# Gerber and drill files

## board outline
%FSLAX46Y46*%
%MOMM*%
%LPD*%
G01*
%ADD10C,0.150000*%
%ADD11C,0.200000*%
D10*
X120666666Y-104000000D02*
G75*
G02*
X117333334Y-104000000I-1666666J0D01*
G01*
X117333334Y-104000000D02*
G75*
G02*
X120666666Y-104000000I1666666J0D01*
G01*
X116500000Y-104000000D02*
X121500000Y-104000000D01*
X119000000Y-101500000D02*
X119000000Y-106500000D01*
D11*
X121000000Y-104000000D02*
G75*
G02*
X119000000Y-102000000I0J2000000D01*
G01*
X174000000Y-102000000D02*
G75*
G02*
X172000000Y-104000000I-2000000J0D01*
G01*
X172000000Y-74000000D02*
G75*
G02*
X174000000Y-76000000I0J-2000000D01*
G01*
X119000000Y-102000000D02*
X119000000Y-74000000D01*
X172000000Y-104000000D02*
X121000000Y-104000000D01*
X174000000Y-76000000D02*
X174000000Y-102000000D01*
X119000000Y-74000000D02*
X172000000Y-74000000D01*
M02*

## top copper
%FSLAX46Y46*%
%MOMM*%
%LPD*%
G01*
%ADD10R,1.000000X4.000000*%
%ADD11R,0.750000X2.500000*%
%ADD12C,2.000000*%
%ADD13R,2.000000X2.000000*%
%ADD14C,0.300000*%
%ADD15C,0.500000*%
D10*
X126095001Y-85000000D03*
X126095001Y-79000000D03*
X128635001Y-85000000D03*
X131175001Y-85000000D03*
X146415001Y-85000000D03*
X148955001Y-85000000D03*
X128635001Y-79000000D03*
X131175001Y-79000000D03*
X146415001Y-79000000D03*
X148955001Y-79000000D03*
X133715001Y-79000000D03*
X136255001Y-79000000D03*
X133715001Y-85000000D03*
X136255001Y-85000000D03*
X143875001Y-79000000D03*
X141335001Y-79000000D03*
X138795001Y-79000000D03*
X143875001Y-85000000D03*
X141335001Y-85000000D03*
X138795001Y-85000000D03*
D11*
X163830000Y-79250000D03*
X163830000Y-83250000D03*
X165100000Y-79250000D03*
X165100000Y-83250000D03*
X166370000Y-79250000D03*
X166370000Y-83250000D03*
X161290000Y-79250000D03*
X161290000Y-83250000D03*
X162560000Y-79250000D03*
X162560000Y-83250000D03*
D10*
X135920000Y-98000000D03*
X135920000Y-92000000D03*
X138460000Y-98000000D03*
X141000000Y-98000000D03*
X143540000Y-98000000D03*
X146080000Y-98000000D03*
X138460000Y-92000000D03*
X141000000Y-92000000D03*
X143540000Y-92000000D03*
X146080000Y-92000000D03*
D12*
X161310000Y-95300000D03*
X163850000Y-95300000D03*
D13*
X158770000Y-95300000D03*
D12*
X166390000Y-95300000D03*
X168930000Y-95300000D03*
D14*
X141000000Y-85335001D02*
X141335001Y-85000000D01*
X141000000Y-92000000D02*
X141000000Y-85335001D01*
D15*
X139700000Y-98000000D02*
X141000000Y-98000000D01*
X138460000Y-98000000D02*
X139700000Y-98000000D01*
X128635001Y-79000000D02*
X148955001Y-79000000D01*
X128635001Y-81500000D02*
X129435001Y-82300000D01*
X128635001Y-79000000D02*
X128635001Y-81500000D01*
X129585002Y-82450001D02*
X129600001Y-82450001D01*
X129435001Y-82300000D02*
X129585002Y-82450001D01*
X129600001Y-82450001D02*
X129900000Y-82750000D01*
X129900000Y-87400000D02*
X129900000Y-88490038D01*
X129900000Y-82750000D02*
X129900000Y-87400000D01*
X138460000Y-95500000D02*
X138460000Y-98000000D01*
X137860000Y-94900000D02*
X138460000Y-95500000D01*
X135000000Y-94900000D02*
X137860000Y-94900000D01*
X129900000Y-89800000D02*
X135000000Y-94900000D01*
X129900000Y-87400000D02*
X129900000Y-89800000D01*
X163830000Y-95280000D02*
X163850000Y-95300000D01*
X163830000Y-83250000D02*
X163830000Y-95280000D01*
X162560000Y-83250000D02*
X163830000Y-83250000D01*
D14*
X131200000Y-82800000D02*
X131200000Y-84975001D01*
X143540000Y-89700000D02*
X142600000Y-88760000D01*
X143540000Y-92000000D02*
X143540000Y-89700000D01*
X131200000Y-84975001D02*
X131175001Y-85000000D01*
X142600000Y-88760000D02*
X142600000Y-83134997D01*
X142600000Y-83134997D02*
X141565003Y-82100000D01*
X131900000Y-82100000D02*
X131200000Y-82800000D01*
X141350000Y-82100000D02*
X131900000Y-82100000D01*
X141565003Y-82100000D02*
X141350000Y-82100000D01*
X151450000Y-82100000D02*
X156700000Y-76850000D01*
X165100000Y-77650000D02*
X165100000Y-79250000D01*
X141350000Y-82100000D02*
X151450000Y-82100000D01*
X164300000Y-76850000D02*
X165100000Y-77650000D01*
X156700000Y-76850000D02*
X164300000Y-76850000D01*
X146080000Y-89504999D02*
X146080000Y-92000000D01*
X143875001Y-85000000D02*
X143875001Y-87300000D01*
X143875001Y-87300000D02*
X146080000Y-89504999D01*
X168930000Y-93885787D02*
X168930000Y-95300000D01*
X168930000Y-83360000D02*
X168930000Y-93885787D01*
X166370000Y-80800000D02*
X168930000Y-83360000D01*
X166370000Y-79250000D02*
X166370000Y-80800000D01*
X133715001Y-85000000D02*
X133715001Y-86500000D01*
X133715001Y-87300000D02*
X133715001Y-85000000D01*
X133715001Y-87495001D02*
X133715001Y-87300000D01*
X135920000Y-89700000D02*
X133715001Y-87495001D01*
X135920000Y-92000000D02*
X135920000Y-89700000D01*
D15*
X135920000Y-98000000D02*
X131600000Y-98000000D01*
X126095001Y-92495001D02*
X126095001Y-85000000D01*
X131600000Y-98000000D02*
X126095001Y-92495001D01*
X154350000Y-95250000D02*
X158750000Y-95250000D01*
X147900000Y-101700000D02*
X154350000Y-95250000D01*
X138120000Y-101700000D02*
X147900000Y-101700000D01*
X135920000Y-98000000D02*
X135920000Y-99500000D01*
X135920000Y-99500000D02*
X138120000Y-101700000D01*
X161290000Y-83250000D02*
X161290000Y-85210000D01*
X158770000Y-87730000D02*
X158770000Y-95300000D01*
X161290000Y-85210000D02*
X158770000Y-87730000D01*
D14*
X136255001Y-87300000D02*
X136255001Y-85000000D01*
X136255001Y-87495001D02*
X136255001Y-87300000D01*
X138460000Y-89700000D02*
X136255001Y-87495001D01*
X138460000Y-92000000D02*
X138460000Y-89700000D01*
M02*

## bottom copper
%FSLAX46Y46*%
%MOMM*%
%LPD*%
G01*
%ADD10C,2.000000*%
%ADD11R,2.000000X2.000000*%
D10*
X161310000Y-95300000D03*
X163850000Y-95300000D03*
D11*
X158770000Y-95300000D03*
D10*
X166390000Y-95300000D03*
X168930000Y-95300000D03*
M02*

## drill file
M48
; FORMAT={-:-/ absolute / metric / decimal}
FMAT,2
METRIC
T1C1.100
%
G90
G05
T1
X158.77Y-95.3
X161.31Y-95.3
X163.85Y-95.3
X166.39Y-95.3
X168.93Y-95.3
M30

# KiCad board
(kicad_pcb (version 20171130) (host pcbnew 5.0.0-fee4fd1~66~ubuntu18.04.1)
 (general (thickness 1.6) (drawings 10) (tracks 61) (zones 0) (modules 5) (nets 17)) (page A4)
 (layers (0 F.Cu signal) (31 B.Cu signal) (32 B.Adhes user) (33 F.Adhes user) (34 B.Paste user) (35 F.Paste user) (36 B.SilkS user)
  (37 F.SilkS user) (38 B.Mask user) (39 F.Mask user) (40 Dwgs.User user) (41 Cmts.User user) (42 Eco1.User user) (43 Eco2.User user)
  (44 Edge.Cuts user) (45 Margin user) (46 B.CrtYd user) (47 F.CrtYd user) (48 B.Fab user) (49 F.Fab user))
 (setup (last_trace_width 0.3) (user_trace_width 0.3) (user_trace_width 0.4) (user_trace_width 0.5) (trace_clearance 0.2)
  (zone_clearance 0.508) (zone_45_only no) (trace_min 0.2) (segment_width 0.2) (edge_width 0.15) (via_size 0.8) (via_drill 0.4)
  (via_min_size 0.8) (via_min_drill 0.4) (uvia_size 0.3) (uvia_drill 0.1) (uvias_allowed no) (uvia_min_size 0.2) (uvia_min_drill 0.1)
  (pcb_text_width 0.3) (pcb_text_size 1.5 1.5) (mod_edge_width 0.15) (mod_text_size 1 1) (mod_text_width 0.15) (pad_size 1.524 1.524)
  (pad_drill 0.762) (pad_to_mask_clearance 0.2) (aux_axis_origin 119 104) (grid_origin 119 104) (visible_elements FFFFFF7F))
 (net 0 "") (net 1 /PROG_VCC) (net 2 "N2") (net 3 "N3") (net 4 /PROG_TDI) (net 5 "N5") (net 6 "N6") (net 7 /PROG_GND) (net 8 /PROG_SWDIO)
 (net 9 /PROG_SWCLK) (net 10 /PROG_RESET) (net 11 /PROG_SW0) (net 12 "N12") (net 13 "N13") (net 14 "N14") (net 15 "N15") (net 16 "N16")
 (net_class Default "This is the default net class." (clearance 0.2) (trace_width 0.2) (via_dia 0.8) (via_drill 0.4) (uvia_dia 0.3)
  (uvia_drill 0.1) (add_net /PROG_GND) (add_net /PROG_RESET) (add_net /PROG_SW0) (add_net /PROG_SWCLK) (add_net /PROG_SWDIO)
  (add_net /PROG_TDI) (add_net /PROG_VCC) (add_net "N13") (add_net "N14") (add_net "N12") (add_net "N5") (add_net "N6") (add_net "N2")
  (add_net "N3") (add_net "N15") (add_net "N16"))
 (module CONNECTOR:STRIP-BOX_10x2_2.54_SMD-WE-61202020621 (layer F.Cu) (at 137.525001 82)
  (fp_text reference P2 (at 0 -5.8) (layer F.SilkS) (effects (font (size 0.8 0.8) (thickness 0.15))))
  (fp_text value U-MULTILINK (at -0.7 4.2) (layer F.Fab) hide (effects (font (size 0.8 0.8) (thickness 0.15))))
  (pad 1 smd rect (at -11.43 3) (size 1 4) (layers F.Cu F.Paste F.Mask) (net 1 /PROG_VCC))
  (pad 2 smd rect (at -11.43 -3) (size 1 4) (layers F.Cu F.Paste F.Mask) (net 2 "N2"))
  (pad 3 smd rect (at -8.89 3) (size 1 4) (layers F.Cu F.Paste F.Mask) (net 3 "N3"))
  (pad 5 smd rect (at -6.35 3) (size 1 4) (layers F.Cu F.Paste F.Mask) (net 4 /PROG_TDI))
  (pad 17 smd rect (at 8.89 3) (size 1 4) (layers F.Cu F.Paste F.Mask) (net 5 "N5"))
  (pad 19 smd rect (at 11.43 3) (size 1 4) (layers F.Cu F.Paste F.Mask) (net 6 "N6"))
  (pad 4 smd rect (at -8.89 -3) (size 1 4) (layers F.Cu F.Paste F.Mask) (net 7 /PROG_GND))
  (pad 6 smd rect (at -6.35 -3) (size 1 4) (layers F.Cu F.Paste F.Mask) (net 7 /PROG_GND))
  (pad 18 smd rect (at 8.89 -3) (size 1 4) (layers F.Cu F.Paste F.Mask) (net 7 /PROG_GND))
  (pad 20 smd rect (at 11.43 -3) (size 1 4) (layers F.Cu F.Paste F.Mask) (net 7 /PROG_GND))
  (pad 8 smd rect (at -3.81 -3) (size 1 4) (layers F.Cu F.Paste F.Mask) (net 7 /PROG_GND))
  (pad 10 smd rect (at -1.27 -3) (size 1 4) (layers F.Cu F.Paste F.Mask) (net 7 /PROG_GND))
  (pad 7 smd rect (at -3.81 3) (size 1 4) (layers F.Cu F.Paste F.Mask) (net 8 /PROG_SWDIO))
  (pad 9 smd rect (at -1.27 3) (size 1 4) (layers F.Cu F.Paste F.Mask) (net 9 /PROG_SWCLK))
  (pad 16 smd rect (at 6.35 -3) (size 1 4) (layers F.Cu F.Paste F.Mask) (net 7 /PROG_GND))
  (pad 14 smd rect (at 3.81 -3) (size 1 4) (layers F.Cu F.Paste F.Mask) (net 7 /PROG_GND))
  (pad 12 smd rect (at 1.27 -3) (size 1 4) (layers F.Cu F.Paste F.Mask) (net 7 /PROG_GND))
  (pad 15 smd rect (at 6.35 3) (size 1 4) (layers F.Cu F.Paste F.Mask) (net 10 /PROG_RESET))
  (pad 13 smd rect (at 3.81 3) (size 1 4) (layers F.Cu F.Paste F.Mask) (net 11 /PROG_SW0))
  (pad 11 smd rect (at 1.27 3) (size 1 4) (layers F.Cu F.Paste F.Mask) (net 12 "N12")))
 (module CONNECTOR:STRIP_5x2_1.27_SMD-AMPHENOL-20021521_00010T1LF (layer F.Cu) (at 163.83 81.25)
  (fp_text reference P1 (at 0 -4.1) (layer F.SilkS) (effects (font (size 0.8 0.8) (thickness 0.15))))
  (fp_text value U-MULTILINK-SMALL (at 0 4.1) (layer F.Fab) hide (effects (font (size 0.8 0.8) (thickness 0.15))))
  (pad 6 smd rect (at 0 -2) (size 0.75 2.5) (layers F.Cu F.Paste F.Mask) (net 11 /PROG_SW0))
  (pad 5 smd rect (at 0 2) (size 0.75 2.5) (layers F.Cu F.Paste F.Mask) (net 7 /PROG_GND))
  (pad 8 smd rect (at 1.27 -2) (size 0.75 2.5) (layers F.Cu F.Paste F.Mask) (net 4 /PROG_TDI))
  (pad 7 smd rect (at 1.27 2) (size 0.75 2.5) (layers F.Cu F.Paste F.Mask) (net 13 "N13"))
  (pad 10 smd rect (at 2.54 -2) (size 0.75 2.5) (layers F.Cu F.Paste F.Mask) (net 10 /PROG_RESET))
  (pad 9 smd rect (at 2.54 2) (size 0.75 2.5) (layers F.Cu F.Paste F.Mask) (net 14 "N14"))
  (pad 2 smd rect (at -2.54 -2) (size 0.75 2.5) (layers F.Cu F.Paste F.Mask) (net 8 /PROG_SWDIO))
  (pad 1 smd rect (at -2.54 2) (size 0.75 2.5) (layers F.Cu F.Paste F.Mask) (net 1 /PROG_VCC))
  (pad 4 smd rect (at -1.27 -2) (size 0.75 2.5) (layers F.Cu F.Paste F.Mask) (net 9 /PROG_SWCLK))
  (pad 3 smd rect (at -1.27 2) (size 0.75 2.5) (layers F.Cu F.Paste F.Mask) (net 7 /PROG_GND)))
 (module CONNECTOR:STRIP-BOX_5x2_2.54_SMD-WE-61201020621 (layer F.Cu) (at 141 95)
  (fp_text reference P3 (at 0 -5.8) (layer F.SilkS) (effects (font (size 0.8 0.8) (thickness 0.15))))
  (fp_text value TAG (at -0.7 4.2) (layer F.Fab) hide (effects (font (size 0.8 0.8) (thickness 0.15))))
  (pad 1 smd rect (at -5.08 3) (size 1 4) (layers F.Cu F.Paste F.Mask) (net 1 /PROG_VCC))
  (pad 2 smd rect (at -5.08 -3) (size 1 4) (layers F.Cu F.Paste F.Mask) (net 8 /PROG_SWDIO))
  (pad 3 smd rect (at -2.54 3) (size 1 4) (layers F.Cu F.Paste F.Mask) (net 7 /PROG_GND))
  (pad 5 smd rect (at 0 3) (size 1 4) (layers F.Cu F.Paste F.Mask) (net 7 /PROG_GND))
  (pad 7 smd rect (at 2.54 3) (size 1 4) (layers F.Cu F.Paste F.Mask) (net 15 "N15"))
  (pad 9 smd rect (at 5.08 3) (size 1 4) (layers F.Cu F.Paste F.Mask) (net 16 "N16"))
  (pad 4 smd rect (at -2.54 -3) (size 1 4) (layers F.Cu F.Paste F.Mask) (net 9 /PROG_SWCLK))
  (pad 6 smd rect (at 0 -3) (size 1 4) (layers F.Cu F.Paste F.Mask) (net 11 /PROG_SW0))
  (pad 8 smd rect (at 2.54 -3) (size 1 4) (layers F.Cu F.Paste F.Mask) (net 4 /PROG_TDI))
  (pad 10 smd rect (at 5.08 -3) (size 1 4) (layers F.Cu F.Paste F.Mask) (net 10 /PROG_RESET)))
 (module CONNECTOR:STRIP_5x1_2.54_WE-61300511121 (layer F.Cu) (at 163.85 95.3)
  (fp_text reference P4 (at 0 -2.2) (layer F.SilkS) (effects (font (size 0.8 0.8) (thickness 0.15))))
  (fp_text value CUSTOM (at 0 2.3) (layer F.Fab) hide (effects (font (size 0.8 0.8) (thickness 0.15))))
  (pad 2 thru_hole circle (at -2.54 0) (size 2 2) (drill 1.1) (layers *.Cu *.Mask) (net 9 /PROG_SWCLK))
  (pad 3 thru_hole circle (at 0 0) (size 2 2) (drill 1.1) (layers *.Cu *.Mask) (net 7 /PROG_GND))
  (pad 1 thru_hole rect (at -5.08 0) (size 2 2) (drill 1.1) (layers *.Cu *.Mask) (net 1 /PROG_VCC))
  (pad 4 thru_hole circle (at 2.54 0) (size 2 2) (drill 1.1) (layers *.Cu *.Mask) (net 8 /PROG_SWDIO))
  (pad 5 thru_hole circle (at 5.08 0) (size 2 2) (drill 1.1) (layers *.Cu *.Mask) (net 10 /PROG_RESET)))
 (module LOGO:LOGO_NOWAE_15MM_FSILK (layer F.Cu) (at 122.35 95.65 90)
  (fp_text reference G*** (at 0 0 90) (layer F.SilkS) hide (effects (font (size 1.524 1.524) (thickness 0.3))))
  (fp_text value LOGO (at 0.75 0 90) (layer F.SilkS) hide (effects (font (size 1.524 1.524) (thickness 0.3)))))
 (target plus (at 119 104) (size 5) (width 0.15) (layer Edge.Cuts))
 (gr_arc (start 121 102) (end 119 102) (angle -90) (layer Edge.Cuts) (width 0.2))
 (gr_arc (start 172 102) (end 172 104) (angle -90) (layer Edge.Cuts) (width 0.2))
 (gr_arc (start 172 76) (end 174 76) (angle -90) (layer Edge.Cuts) (width 0.2))
 (gr_line (start 119 102) (end 119 74) (layer Edge.Cuts) (width 0.2))
 (gr_line (start 172 104) (end 121 104) (layer Edge.Cuts) (width 0.2))
 (gr_line (start 174 76) (end 174 102) (layer Edge.Cuts) (width 0.2))
 (gr_line (start 119 74) (end 172 74) (layer Edge.Cuts) (width 0.2))
 (segment (start 141 85.335001) (end 141.335001 85) (width 0.3) (layer F.Cu) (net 11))
 (segment (start 141 92) (end 141 85.335001) (width 0.3) (layer F.Cu) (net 11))
 (segment (start 139.7 98) (end 141 98) (width 0.5) (layer F.Cu) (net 7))
 (segment (start 138.46 98) (end 139.7 98) (width 0.5) (layer F.Cu) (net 7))
 (segment (start 128.635001 79) (end 148.955001 79) (width 0.5) (layer F.Cu) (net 7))
 (segment (start 128.635001 81.5) (end 129.435001 82.3) (width 0.5) (layer F.Cu) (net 7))
 (segment (start 128.635001 79) (end 128.635001 81.5) (width 0.5) (layer F.Cu) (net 7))
 (segment (start 129.585002 82.450001) (end 129.600001 82.450001) (width 0.5) (layer F.Cu) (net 7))
 (segment (start 129.435001 82.3) (end 129.585002 82.450001) (width 0.5) (layer F.Cu) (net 7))
 (segment (start 129.600001 82.450001) (end 129.9 82.75) (width 0.5) (layer F.Cu) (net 7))
 (segment (start 129.9 87.4) (end 129.9 88.490038) (width 0.5) (layer F.Cu) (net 7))
 (segment (start 129.9 82.75) (end 129.9 87.4) (width 0.5) (layer F.Cu) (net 7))
 (segment (start 138.46 95.5) (end 138.46 98) (width 0.5) (layer F.Cu) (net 7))
 (segment (start 137.86 94.9) (end 138.46 95.5) (width 0.5) (layer F.Cu) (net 7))
 (segment (start 135 94.9) (end 137.86 94.9) (width 0.5) (layer F.Cu) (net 7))
 (segment (start 129.9 89.8) (end 135 94.9) (width 0.5) (layer F.Cu) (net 7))
 (segment (start 129.9 87.4) (end 129.9 89.8) (width 0.5) (layer F.Cu) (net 7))
 (segment (start 163.83 95.28) (end 163.85 95.3) (width 0.5) (layer F.Cu) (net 7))
 (segment (start 163.83 83.25) (end 163.83 95.28) (width 0.5) (layer F.Cu) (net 7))
 (segment (start 162.56 83.25) (end 163.83 83.25) (width 0.5) (layer F.Cu) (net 7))
 (segment (start 131.2 82.8) (end 131.2 84.975001) (width 0.3) (layer F.Cu) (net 4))
 (segment (start 143.54 89.7) (end 142.6 88.76) (width 0.3) (layer F.Cu) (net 4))
 (segment (start 143.54 92) (end 143.54 89.7) (width 0.3) (layer F.Cu) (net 4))
 (segment (start 131.2 84.975001) (end 131.175001 85) (width 0.3) (layer F.Cu) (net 4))
 (segment (start 142.6 88.76) (end 142.6 83.134997) (width 0.3) (layer F.Cu) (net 4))
 (segment (start 142.6 83.134997) (end 141.565003 82.1) (width 0.3) (layer F.Cu) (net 4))
 (segment (start 131.9 82.1) (end 131.2 82.8) (width 0.3) (layer F.Cu) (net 4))
 (segment (start 141.35 82.1) (end 131.9 82.1) (width 0.3) (layer F.Cu) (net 4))
 (segment (start 141.565003 82.1) (end 141.35 82.1) (width 0.3) (layer F.Cu) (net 4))
 (segment (start 151.45 82.1) (end 156.7 76.85) (width 0.3) (layer F.Cu) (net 4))
 (segment (start 165.1 77.65) (end 165.1 79.25) (width 0.3) (layer F.Cu) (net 4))
 (segment (start 141.35 82.1) (end 151.45 82.1) (width 0.3) (layer F.Cu) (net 4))
 (segment (start 164.3 76.85) (end 165.1 77.65) (width 0.3) (layer F.Cu) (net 4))
 (segment (start 156.7 76.85) (end 164.3 76.85) (width 0.3) (layer F.Cu) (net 4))
 (segment (start 146.08 89.504999) (end 146.08 92) (width 0.3) (layer F.Cu) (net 10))
 (segment (start 143.875001 85) (end 143.875001 87.3) (width 0.3) (layer F.Cu) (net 10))
 (segment (start 143.875001 87.3) (end 146.08 89.504999) (width 0.3) (layer F.Cu) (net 10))
 (segment (start 168.93 93.885787) (end 168.93 95.3) (width 0.3) (layer F.Cu) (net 10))
 (segment (start 168.93 83.36) (end 168.93 93.885787) (width 0.3) (layer F.Cu) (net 10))
 (segment (start 166.37 80.8) (end 168.93 83.36) (width 0.3) (layer F.Cu) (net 10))
 (segment (start 166.37 79.25) (end 166.37 80.8) (width 0.3) (layer F.Cu) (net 10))
 (segment (start 133.715001 85) (end 133.715001 86.5) (width 0.3) (layer F.Cu) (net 8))
 (segment (start 133.715001 87.3) (end 133.715001 85) (width 0.3) (layer F.Cu) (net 8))
 (segment (start 133.715001 87.495001) (end 133.715001 87.3) (width 0.3) (layer F.Cu) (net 8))
 (segment (start 135.92 89.7) (end 133.715001 87.495001) (width 0.3) (layer F.Cu) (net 8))
 (segment (start 135.92 92) (end 135.92 89.7) (width 0.3) (layer F.Cu) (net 8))
 (segment (start 135.92 98) (end 131.6 98) (width 0.5) (layer F.Cu) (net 1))
 (segment (start 126.095001 92.495001) (end 126.095001 85) (width 0.5) (layer F.Cu) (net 1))
 (segment (start 131.6 98) (end 126.095001 92.495001) (width 0.5) (layer F.Cu) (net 1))
 (segment (start 154.35 95.25) (end 158.75 95.25) (width 0.5) (layer F.Cu) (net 1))
 (segment (start 147.9 101.7) (end 154.35 95.25) (width 0.5) (layer F.Cu) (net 1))
 (segment (start 138.12 101.7) (end 147.9 101.7) (width 0.5) (layer F.Cu) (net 1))
 (segment (start 135.92 98) (end 135.92 99.5) (width 0.5) (layer F.Cu) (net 1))
 (segment (start 135.92 99.5) (end 138.12 101.7) (width 0.5) (layer F.Cu) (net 1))
 (segment (start 161.29 83.25) (end 161.29 85.21) (width 0.5) (layer F.Cu) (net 1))
 (segment (start 158.77 87.73) (end 158.77 95.3) (width 0.5) (layer F.Cu) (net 1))
 (segment (start 161.29 85.21) (end 158.77 87.73) (width 0.5) (layer F.Cu) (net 1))
 (segment (start 136.255001 87.3) (end 136.255001 85) (width 0.3) (layer F.Cu) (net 9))
 (segment (start 136.255001 87.495001) (end 136.255001 87.3) (width 0.3) (layer F.Cu) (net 9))
 (segment (start 138.46 89.7) (end 136.255001 87.495001) (width 0.3) (layer F.Cu) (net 9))
 (segment (start 138.46 92) (end 138.46 89.7) (width 0.3) (layer F.Cu) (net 9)))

